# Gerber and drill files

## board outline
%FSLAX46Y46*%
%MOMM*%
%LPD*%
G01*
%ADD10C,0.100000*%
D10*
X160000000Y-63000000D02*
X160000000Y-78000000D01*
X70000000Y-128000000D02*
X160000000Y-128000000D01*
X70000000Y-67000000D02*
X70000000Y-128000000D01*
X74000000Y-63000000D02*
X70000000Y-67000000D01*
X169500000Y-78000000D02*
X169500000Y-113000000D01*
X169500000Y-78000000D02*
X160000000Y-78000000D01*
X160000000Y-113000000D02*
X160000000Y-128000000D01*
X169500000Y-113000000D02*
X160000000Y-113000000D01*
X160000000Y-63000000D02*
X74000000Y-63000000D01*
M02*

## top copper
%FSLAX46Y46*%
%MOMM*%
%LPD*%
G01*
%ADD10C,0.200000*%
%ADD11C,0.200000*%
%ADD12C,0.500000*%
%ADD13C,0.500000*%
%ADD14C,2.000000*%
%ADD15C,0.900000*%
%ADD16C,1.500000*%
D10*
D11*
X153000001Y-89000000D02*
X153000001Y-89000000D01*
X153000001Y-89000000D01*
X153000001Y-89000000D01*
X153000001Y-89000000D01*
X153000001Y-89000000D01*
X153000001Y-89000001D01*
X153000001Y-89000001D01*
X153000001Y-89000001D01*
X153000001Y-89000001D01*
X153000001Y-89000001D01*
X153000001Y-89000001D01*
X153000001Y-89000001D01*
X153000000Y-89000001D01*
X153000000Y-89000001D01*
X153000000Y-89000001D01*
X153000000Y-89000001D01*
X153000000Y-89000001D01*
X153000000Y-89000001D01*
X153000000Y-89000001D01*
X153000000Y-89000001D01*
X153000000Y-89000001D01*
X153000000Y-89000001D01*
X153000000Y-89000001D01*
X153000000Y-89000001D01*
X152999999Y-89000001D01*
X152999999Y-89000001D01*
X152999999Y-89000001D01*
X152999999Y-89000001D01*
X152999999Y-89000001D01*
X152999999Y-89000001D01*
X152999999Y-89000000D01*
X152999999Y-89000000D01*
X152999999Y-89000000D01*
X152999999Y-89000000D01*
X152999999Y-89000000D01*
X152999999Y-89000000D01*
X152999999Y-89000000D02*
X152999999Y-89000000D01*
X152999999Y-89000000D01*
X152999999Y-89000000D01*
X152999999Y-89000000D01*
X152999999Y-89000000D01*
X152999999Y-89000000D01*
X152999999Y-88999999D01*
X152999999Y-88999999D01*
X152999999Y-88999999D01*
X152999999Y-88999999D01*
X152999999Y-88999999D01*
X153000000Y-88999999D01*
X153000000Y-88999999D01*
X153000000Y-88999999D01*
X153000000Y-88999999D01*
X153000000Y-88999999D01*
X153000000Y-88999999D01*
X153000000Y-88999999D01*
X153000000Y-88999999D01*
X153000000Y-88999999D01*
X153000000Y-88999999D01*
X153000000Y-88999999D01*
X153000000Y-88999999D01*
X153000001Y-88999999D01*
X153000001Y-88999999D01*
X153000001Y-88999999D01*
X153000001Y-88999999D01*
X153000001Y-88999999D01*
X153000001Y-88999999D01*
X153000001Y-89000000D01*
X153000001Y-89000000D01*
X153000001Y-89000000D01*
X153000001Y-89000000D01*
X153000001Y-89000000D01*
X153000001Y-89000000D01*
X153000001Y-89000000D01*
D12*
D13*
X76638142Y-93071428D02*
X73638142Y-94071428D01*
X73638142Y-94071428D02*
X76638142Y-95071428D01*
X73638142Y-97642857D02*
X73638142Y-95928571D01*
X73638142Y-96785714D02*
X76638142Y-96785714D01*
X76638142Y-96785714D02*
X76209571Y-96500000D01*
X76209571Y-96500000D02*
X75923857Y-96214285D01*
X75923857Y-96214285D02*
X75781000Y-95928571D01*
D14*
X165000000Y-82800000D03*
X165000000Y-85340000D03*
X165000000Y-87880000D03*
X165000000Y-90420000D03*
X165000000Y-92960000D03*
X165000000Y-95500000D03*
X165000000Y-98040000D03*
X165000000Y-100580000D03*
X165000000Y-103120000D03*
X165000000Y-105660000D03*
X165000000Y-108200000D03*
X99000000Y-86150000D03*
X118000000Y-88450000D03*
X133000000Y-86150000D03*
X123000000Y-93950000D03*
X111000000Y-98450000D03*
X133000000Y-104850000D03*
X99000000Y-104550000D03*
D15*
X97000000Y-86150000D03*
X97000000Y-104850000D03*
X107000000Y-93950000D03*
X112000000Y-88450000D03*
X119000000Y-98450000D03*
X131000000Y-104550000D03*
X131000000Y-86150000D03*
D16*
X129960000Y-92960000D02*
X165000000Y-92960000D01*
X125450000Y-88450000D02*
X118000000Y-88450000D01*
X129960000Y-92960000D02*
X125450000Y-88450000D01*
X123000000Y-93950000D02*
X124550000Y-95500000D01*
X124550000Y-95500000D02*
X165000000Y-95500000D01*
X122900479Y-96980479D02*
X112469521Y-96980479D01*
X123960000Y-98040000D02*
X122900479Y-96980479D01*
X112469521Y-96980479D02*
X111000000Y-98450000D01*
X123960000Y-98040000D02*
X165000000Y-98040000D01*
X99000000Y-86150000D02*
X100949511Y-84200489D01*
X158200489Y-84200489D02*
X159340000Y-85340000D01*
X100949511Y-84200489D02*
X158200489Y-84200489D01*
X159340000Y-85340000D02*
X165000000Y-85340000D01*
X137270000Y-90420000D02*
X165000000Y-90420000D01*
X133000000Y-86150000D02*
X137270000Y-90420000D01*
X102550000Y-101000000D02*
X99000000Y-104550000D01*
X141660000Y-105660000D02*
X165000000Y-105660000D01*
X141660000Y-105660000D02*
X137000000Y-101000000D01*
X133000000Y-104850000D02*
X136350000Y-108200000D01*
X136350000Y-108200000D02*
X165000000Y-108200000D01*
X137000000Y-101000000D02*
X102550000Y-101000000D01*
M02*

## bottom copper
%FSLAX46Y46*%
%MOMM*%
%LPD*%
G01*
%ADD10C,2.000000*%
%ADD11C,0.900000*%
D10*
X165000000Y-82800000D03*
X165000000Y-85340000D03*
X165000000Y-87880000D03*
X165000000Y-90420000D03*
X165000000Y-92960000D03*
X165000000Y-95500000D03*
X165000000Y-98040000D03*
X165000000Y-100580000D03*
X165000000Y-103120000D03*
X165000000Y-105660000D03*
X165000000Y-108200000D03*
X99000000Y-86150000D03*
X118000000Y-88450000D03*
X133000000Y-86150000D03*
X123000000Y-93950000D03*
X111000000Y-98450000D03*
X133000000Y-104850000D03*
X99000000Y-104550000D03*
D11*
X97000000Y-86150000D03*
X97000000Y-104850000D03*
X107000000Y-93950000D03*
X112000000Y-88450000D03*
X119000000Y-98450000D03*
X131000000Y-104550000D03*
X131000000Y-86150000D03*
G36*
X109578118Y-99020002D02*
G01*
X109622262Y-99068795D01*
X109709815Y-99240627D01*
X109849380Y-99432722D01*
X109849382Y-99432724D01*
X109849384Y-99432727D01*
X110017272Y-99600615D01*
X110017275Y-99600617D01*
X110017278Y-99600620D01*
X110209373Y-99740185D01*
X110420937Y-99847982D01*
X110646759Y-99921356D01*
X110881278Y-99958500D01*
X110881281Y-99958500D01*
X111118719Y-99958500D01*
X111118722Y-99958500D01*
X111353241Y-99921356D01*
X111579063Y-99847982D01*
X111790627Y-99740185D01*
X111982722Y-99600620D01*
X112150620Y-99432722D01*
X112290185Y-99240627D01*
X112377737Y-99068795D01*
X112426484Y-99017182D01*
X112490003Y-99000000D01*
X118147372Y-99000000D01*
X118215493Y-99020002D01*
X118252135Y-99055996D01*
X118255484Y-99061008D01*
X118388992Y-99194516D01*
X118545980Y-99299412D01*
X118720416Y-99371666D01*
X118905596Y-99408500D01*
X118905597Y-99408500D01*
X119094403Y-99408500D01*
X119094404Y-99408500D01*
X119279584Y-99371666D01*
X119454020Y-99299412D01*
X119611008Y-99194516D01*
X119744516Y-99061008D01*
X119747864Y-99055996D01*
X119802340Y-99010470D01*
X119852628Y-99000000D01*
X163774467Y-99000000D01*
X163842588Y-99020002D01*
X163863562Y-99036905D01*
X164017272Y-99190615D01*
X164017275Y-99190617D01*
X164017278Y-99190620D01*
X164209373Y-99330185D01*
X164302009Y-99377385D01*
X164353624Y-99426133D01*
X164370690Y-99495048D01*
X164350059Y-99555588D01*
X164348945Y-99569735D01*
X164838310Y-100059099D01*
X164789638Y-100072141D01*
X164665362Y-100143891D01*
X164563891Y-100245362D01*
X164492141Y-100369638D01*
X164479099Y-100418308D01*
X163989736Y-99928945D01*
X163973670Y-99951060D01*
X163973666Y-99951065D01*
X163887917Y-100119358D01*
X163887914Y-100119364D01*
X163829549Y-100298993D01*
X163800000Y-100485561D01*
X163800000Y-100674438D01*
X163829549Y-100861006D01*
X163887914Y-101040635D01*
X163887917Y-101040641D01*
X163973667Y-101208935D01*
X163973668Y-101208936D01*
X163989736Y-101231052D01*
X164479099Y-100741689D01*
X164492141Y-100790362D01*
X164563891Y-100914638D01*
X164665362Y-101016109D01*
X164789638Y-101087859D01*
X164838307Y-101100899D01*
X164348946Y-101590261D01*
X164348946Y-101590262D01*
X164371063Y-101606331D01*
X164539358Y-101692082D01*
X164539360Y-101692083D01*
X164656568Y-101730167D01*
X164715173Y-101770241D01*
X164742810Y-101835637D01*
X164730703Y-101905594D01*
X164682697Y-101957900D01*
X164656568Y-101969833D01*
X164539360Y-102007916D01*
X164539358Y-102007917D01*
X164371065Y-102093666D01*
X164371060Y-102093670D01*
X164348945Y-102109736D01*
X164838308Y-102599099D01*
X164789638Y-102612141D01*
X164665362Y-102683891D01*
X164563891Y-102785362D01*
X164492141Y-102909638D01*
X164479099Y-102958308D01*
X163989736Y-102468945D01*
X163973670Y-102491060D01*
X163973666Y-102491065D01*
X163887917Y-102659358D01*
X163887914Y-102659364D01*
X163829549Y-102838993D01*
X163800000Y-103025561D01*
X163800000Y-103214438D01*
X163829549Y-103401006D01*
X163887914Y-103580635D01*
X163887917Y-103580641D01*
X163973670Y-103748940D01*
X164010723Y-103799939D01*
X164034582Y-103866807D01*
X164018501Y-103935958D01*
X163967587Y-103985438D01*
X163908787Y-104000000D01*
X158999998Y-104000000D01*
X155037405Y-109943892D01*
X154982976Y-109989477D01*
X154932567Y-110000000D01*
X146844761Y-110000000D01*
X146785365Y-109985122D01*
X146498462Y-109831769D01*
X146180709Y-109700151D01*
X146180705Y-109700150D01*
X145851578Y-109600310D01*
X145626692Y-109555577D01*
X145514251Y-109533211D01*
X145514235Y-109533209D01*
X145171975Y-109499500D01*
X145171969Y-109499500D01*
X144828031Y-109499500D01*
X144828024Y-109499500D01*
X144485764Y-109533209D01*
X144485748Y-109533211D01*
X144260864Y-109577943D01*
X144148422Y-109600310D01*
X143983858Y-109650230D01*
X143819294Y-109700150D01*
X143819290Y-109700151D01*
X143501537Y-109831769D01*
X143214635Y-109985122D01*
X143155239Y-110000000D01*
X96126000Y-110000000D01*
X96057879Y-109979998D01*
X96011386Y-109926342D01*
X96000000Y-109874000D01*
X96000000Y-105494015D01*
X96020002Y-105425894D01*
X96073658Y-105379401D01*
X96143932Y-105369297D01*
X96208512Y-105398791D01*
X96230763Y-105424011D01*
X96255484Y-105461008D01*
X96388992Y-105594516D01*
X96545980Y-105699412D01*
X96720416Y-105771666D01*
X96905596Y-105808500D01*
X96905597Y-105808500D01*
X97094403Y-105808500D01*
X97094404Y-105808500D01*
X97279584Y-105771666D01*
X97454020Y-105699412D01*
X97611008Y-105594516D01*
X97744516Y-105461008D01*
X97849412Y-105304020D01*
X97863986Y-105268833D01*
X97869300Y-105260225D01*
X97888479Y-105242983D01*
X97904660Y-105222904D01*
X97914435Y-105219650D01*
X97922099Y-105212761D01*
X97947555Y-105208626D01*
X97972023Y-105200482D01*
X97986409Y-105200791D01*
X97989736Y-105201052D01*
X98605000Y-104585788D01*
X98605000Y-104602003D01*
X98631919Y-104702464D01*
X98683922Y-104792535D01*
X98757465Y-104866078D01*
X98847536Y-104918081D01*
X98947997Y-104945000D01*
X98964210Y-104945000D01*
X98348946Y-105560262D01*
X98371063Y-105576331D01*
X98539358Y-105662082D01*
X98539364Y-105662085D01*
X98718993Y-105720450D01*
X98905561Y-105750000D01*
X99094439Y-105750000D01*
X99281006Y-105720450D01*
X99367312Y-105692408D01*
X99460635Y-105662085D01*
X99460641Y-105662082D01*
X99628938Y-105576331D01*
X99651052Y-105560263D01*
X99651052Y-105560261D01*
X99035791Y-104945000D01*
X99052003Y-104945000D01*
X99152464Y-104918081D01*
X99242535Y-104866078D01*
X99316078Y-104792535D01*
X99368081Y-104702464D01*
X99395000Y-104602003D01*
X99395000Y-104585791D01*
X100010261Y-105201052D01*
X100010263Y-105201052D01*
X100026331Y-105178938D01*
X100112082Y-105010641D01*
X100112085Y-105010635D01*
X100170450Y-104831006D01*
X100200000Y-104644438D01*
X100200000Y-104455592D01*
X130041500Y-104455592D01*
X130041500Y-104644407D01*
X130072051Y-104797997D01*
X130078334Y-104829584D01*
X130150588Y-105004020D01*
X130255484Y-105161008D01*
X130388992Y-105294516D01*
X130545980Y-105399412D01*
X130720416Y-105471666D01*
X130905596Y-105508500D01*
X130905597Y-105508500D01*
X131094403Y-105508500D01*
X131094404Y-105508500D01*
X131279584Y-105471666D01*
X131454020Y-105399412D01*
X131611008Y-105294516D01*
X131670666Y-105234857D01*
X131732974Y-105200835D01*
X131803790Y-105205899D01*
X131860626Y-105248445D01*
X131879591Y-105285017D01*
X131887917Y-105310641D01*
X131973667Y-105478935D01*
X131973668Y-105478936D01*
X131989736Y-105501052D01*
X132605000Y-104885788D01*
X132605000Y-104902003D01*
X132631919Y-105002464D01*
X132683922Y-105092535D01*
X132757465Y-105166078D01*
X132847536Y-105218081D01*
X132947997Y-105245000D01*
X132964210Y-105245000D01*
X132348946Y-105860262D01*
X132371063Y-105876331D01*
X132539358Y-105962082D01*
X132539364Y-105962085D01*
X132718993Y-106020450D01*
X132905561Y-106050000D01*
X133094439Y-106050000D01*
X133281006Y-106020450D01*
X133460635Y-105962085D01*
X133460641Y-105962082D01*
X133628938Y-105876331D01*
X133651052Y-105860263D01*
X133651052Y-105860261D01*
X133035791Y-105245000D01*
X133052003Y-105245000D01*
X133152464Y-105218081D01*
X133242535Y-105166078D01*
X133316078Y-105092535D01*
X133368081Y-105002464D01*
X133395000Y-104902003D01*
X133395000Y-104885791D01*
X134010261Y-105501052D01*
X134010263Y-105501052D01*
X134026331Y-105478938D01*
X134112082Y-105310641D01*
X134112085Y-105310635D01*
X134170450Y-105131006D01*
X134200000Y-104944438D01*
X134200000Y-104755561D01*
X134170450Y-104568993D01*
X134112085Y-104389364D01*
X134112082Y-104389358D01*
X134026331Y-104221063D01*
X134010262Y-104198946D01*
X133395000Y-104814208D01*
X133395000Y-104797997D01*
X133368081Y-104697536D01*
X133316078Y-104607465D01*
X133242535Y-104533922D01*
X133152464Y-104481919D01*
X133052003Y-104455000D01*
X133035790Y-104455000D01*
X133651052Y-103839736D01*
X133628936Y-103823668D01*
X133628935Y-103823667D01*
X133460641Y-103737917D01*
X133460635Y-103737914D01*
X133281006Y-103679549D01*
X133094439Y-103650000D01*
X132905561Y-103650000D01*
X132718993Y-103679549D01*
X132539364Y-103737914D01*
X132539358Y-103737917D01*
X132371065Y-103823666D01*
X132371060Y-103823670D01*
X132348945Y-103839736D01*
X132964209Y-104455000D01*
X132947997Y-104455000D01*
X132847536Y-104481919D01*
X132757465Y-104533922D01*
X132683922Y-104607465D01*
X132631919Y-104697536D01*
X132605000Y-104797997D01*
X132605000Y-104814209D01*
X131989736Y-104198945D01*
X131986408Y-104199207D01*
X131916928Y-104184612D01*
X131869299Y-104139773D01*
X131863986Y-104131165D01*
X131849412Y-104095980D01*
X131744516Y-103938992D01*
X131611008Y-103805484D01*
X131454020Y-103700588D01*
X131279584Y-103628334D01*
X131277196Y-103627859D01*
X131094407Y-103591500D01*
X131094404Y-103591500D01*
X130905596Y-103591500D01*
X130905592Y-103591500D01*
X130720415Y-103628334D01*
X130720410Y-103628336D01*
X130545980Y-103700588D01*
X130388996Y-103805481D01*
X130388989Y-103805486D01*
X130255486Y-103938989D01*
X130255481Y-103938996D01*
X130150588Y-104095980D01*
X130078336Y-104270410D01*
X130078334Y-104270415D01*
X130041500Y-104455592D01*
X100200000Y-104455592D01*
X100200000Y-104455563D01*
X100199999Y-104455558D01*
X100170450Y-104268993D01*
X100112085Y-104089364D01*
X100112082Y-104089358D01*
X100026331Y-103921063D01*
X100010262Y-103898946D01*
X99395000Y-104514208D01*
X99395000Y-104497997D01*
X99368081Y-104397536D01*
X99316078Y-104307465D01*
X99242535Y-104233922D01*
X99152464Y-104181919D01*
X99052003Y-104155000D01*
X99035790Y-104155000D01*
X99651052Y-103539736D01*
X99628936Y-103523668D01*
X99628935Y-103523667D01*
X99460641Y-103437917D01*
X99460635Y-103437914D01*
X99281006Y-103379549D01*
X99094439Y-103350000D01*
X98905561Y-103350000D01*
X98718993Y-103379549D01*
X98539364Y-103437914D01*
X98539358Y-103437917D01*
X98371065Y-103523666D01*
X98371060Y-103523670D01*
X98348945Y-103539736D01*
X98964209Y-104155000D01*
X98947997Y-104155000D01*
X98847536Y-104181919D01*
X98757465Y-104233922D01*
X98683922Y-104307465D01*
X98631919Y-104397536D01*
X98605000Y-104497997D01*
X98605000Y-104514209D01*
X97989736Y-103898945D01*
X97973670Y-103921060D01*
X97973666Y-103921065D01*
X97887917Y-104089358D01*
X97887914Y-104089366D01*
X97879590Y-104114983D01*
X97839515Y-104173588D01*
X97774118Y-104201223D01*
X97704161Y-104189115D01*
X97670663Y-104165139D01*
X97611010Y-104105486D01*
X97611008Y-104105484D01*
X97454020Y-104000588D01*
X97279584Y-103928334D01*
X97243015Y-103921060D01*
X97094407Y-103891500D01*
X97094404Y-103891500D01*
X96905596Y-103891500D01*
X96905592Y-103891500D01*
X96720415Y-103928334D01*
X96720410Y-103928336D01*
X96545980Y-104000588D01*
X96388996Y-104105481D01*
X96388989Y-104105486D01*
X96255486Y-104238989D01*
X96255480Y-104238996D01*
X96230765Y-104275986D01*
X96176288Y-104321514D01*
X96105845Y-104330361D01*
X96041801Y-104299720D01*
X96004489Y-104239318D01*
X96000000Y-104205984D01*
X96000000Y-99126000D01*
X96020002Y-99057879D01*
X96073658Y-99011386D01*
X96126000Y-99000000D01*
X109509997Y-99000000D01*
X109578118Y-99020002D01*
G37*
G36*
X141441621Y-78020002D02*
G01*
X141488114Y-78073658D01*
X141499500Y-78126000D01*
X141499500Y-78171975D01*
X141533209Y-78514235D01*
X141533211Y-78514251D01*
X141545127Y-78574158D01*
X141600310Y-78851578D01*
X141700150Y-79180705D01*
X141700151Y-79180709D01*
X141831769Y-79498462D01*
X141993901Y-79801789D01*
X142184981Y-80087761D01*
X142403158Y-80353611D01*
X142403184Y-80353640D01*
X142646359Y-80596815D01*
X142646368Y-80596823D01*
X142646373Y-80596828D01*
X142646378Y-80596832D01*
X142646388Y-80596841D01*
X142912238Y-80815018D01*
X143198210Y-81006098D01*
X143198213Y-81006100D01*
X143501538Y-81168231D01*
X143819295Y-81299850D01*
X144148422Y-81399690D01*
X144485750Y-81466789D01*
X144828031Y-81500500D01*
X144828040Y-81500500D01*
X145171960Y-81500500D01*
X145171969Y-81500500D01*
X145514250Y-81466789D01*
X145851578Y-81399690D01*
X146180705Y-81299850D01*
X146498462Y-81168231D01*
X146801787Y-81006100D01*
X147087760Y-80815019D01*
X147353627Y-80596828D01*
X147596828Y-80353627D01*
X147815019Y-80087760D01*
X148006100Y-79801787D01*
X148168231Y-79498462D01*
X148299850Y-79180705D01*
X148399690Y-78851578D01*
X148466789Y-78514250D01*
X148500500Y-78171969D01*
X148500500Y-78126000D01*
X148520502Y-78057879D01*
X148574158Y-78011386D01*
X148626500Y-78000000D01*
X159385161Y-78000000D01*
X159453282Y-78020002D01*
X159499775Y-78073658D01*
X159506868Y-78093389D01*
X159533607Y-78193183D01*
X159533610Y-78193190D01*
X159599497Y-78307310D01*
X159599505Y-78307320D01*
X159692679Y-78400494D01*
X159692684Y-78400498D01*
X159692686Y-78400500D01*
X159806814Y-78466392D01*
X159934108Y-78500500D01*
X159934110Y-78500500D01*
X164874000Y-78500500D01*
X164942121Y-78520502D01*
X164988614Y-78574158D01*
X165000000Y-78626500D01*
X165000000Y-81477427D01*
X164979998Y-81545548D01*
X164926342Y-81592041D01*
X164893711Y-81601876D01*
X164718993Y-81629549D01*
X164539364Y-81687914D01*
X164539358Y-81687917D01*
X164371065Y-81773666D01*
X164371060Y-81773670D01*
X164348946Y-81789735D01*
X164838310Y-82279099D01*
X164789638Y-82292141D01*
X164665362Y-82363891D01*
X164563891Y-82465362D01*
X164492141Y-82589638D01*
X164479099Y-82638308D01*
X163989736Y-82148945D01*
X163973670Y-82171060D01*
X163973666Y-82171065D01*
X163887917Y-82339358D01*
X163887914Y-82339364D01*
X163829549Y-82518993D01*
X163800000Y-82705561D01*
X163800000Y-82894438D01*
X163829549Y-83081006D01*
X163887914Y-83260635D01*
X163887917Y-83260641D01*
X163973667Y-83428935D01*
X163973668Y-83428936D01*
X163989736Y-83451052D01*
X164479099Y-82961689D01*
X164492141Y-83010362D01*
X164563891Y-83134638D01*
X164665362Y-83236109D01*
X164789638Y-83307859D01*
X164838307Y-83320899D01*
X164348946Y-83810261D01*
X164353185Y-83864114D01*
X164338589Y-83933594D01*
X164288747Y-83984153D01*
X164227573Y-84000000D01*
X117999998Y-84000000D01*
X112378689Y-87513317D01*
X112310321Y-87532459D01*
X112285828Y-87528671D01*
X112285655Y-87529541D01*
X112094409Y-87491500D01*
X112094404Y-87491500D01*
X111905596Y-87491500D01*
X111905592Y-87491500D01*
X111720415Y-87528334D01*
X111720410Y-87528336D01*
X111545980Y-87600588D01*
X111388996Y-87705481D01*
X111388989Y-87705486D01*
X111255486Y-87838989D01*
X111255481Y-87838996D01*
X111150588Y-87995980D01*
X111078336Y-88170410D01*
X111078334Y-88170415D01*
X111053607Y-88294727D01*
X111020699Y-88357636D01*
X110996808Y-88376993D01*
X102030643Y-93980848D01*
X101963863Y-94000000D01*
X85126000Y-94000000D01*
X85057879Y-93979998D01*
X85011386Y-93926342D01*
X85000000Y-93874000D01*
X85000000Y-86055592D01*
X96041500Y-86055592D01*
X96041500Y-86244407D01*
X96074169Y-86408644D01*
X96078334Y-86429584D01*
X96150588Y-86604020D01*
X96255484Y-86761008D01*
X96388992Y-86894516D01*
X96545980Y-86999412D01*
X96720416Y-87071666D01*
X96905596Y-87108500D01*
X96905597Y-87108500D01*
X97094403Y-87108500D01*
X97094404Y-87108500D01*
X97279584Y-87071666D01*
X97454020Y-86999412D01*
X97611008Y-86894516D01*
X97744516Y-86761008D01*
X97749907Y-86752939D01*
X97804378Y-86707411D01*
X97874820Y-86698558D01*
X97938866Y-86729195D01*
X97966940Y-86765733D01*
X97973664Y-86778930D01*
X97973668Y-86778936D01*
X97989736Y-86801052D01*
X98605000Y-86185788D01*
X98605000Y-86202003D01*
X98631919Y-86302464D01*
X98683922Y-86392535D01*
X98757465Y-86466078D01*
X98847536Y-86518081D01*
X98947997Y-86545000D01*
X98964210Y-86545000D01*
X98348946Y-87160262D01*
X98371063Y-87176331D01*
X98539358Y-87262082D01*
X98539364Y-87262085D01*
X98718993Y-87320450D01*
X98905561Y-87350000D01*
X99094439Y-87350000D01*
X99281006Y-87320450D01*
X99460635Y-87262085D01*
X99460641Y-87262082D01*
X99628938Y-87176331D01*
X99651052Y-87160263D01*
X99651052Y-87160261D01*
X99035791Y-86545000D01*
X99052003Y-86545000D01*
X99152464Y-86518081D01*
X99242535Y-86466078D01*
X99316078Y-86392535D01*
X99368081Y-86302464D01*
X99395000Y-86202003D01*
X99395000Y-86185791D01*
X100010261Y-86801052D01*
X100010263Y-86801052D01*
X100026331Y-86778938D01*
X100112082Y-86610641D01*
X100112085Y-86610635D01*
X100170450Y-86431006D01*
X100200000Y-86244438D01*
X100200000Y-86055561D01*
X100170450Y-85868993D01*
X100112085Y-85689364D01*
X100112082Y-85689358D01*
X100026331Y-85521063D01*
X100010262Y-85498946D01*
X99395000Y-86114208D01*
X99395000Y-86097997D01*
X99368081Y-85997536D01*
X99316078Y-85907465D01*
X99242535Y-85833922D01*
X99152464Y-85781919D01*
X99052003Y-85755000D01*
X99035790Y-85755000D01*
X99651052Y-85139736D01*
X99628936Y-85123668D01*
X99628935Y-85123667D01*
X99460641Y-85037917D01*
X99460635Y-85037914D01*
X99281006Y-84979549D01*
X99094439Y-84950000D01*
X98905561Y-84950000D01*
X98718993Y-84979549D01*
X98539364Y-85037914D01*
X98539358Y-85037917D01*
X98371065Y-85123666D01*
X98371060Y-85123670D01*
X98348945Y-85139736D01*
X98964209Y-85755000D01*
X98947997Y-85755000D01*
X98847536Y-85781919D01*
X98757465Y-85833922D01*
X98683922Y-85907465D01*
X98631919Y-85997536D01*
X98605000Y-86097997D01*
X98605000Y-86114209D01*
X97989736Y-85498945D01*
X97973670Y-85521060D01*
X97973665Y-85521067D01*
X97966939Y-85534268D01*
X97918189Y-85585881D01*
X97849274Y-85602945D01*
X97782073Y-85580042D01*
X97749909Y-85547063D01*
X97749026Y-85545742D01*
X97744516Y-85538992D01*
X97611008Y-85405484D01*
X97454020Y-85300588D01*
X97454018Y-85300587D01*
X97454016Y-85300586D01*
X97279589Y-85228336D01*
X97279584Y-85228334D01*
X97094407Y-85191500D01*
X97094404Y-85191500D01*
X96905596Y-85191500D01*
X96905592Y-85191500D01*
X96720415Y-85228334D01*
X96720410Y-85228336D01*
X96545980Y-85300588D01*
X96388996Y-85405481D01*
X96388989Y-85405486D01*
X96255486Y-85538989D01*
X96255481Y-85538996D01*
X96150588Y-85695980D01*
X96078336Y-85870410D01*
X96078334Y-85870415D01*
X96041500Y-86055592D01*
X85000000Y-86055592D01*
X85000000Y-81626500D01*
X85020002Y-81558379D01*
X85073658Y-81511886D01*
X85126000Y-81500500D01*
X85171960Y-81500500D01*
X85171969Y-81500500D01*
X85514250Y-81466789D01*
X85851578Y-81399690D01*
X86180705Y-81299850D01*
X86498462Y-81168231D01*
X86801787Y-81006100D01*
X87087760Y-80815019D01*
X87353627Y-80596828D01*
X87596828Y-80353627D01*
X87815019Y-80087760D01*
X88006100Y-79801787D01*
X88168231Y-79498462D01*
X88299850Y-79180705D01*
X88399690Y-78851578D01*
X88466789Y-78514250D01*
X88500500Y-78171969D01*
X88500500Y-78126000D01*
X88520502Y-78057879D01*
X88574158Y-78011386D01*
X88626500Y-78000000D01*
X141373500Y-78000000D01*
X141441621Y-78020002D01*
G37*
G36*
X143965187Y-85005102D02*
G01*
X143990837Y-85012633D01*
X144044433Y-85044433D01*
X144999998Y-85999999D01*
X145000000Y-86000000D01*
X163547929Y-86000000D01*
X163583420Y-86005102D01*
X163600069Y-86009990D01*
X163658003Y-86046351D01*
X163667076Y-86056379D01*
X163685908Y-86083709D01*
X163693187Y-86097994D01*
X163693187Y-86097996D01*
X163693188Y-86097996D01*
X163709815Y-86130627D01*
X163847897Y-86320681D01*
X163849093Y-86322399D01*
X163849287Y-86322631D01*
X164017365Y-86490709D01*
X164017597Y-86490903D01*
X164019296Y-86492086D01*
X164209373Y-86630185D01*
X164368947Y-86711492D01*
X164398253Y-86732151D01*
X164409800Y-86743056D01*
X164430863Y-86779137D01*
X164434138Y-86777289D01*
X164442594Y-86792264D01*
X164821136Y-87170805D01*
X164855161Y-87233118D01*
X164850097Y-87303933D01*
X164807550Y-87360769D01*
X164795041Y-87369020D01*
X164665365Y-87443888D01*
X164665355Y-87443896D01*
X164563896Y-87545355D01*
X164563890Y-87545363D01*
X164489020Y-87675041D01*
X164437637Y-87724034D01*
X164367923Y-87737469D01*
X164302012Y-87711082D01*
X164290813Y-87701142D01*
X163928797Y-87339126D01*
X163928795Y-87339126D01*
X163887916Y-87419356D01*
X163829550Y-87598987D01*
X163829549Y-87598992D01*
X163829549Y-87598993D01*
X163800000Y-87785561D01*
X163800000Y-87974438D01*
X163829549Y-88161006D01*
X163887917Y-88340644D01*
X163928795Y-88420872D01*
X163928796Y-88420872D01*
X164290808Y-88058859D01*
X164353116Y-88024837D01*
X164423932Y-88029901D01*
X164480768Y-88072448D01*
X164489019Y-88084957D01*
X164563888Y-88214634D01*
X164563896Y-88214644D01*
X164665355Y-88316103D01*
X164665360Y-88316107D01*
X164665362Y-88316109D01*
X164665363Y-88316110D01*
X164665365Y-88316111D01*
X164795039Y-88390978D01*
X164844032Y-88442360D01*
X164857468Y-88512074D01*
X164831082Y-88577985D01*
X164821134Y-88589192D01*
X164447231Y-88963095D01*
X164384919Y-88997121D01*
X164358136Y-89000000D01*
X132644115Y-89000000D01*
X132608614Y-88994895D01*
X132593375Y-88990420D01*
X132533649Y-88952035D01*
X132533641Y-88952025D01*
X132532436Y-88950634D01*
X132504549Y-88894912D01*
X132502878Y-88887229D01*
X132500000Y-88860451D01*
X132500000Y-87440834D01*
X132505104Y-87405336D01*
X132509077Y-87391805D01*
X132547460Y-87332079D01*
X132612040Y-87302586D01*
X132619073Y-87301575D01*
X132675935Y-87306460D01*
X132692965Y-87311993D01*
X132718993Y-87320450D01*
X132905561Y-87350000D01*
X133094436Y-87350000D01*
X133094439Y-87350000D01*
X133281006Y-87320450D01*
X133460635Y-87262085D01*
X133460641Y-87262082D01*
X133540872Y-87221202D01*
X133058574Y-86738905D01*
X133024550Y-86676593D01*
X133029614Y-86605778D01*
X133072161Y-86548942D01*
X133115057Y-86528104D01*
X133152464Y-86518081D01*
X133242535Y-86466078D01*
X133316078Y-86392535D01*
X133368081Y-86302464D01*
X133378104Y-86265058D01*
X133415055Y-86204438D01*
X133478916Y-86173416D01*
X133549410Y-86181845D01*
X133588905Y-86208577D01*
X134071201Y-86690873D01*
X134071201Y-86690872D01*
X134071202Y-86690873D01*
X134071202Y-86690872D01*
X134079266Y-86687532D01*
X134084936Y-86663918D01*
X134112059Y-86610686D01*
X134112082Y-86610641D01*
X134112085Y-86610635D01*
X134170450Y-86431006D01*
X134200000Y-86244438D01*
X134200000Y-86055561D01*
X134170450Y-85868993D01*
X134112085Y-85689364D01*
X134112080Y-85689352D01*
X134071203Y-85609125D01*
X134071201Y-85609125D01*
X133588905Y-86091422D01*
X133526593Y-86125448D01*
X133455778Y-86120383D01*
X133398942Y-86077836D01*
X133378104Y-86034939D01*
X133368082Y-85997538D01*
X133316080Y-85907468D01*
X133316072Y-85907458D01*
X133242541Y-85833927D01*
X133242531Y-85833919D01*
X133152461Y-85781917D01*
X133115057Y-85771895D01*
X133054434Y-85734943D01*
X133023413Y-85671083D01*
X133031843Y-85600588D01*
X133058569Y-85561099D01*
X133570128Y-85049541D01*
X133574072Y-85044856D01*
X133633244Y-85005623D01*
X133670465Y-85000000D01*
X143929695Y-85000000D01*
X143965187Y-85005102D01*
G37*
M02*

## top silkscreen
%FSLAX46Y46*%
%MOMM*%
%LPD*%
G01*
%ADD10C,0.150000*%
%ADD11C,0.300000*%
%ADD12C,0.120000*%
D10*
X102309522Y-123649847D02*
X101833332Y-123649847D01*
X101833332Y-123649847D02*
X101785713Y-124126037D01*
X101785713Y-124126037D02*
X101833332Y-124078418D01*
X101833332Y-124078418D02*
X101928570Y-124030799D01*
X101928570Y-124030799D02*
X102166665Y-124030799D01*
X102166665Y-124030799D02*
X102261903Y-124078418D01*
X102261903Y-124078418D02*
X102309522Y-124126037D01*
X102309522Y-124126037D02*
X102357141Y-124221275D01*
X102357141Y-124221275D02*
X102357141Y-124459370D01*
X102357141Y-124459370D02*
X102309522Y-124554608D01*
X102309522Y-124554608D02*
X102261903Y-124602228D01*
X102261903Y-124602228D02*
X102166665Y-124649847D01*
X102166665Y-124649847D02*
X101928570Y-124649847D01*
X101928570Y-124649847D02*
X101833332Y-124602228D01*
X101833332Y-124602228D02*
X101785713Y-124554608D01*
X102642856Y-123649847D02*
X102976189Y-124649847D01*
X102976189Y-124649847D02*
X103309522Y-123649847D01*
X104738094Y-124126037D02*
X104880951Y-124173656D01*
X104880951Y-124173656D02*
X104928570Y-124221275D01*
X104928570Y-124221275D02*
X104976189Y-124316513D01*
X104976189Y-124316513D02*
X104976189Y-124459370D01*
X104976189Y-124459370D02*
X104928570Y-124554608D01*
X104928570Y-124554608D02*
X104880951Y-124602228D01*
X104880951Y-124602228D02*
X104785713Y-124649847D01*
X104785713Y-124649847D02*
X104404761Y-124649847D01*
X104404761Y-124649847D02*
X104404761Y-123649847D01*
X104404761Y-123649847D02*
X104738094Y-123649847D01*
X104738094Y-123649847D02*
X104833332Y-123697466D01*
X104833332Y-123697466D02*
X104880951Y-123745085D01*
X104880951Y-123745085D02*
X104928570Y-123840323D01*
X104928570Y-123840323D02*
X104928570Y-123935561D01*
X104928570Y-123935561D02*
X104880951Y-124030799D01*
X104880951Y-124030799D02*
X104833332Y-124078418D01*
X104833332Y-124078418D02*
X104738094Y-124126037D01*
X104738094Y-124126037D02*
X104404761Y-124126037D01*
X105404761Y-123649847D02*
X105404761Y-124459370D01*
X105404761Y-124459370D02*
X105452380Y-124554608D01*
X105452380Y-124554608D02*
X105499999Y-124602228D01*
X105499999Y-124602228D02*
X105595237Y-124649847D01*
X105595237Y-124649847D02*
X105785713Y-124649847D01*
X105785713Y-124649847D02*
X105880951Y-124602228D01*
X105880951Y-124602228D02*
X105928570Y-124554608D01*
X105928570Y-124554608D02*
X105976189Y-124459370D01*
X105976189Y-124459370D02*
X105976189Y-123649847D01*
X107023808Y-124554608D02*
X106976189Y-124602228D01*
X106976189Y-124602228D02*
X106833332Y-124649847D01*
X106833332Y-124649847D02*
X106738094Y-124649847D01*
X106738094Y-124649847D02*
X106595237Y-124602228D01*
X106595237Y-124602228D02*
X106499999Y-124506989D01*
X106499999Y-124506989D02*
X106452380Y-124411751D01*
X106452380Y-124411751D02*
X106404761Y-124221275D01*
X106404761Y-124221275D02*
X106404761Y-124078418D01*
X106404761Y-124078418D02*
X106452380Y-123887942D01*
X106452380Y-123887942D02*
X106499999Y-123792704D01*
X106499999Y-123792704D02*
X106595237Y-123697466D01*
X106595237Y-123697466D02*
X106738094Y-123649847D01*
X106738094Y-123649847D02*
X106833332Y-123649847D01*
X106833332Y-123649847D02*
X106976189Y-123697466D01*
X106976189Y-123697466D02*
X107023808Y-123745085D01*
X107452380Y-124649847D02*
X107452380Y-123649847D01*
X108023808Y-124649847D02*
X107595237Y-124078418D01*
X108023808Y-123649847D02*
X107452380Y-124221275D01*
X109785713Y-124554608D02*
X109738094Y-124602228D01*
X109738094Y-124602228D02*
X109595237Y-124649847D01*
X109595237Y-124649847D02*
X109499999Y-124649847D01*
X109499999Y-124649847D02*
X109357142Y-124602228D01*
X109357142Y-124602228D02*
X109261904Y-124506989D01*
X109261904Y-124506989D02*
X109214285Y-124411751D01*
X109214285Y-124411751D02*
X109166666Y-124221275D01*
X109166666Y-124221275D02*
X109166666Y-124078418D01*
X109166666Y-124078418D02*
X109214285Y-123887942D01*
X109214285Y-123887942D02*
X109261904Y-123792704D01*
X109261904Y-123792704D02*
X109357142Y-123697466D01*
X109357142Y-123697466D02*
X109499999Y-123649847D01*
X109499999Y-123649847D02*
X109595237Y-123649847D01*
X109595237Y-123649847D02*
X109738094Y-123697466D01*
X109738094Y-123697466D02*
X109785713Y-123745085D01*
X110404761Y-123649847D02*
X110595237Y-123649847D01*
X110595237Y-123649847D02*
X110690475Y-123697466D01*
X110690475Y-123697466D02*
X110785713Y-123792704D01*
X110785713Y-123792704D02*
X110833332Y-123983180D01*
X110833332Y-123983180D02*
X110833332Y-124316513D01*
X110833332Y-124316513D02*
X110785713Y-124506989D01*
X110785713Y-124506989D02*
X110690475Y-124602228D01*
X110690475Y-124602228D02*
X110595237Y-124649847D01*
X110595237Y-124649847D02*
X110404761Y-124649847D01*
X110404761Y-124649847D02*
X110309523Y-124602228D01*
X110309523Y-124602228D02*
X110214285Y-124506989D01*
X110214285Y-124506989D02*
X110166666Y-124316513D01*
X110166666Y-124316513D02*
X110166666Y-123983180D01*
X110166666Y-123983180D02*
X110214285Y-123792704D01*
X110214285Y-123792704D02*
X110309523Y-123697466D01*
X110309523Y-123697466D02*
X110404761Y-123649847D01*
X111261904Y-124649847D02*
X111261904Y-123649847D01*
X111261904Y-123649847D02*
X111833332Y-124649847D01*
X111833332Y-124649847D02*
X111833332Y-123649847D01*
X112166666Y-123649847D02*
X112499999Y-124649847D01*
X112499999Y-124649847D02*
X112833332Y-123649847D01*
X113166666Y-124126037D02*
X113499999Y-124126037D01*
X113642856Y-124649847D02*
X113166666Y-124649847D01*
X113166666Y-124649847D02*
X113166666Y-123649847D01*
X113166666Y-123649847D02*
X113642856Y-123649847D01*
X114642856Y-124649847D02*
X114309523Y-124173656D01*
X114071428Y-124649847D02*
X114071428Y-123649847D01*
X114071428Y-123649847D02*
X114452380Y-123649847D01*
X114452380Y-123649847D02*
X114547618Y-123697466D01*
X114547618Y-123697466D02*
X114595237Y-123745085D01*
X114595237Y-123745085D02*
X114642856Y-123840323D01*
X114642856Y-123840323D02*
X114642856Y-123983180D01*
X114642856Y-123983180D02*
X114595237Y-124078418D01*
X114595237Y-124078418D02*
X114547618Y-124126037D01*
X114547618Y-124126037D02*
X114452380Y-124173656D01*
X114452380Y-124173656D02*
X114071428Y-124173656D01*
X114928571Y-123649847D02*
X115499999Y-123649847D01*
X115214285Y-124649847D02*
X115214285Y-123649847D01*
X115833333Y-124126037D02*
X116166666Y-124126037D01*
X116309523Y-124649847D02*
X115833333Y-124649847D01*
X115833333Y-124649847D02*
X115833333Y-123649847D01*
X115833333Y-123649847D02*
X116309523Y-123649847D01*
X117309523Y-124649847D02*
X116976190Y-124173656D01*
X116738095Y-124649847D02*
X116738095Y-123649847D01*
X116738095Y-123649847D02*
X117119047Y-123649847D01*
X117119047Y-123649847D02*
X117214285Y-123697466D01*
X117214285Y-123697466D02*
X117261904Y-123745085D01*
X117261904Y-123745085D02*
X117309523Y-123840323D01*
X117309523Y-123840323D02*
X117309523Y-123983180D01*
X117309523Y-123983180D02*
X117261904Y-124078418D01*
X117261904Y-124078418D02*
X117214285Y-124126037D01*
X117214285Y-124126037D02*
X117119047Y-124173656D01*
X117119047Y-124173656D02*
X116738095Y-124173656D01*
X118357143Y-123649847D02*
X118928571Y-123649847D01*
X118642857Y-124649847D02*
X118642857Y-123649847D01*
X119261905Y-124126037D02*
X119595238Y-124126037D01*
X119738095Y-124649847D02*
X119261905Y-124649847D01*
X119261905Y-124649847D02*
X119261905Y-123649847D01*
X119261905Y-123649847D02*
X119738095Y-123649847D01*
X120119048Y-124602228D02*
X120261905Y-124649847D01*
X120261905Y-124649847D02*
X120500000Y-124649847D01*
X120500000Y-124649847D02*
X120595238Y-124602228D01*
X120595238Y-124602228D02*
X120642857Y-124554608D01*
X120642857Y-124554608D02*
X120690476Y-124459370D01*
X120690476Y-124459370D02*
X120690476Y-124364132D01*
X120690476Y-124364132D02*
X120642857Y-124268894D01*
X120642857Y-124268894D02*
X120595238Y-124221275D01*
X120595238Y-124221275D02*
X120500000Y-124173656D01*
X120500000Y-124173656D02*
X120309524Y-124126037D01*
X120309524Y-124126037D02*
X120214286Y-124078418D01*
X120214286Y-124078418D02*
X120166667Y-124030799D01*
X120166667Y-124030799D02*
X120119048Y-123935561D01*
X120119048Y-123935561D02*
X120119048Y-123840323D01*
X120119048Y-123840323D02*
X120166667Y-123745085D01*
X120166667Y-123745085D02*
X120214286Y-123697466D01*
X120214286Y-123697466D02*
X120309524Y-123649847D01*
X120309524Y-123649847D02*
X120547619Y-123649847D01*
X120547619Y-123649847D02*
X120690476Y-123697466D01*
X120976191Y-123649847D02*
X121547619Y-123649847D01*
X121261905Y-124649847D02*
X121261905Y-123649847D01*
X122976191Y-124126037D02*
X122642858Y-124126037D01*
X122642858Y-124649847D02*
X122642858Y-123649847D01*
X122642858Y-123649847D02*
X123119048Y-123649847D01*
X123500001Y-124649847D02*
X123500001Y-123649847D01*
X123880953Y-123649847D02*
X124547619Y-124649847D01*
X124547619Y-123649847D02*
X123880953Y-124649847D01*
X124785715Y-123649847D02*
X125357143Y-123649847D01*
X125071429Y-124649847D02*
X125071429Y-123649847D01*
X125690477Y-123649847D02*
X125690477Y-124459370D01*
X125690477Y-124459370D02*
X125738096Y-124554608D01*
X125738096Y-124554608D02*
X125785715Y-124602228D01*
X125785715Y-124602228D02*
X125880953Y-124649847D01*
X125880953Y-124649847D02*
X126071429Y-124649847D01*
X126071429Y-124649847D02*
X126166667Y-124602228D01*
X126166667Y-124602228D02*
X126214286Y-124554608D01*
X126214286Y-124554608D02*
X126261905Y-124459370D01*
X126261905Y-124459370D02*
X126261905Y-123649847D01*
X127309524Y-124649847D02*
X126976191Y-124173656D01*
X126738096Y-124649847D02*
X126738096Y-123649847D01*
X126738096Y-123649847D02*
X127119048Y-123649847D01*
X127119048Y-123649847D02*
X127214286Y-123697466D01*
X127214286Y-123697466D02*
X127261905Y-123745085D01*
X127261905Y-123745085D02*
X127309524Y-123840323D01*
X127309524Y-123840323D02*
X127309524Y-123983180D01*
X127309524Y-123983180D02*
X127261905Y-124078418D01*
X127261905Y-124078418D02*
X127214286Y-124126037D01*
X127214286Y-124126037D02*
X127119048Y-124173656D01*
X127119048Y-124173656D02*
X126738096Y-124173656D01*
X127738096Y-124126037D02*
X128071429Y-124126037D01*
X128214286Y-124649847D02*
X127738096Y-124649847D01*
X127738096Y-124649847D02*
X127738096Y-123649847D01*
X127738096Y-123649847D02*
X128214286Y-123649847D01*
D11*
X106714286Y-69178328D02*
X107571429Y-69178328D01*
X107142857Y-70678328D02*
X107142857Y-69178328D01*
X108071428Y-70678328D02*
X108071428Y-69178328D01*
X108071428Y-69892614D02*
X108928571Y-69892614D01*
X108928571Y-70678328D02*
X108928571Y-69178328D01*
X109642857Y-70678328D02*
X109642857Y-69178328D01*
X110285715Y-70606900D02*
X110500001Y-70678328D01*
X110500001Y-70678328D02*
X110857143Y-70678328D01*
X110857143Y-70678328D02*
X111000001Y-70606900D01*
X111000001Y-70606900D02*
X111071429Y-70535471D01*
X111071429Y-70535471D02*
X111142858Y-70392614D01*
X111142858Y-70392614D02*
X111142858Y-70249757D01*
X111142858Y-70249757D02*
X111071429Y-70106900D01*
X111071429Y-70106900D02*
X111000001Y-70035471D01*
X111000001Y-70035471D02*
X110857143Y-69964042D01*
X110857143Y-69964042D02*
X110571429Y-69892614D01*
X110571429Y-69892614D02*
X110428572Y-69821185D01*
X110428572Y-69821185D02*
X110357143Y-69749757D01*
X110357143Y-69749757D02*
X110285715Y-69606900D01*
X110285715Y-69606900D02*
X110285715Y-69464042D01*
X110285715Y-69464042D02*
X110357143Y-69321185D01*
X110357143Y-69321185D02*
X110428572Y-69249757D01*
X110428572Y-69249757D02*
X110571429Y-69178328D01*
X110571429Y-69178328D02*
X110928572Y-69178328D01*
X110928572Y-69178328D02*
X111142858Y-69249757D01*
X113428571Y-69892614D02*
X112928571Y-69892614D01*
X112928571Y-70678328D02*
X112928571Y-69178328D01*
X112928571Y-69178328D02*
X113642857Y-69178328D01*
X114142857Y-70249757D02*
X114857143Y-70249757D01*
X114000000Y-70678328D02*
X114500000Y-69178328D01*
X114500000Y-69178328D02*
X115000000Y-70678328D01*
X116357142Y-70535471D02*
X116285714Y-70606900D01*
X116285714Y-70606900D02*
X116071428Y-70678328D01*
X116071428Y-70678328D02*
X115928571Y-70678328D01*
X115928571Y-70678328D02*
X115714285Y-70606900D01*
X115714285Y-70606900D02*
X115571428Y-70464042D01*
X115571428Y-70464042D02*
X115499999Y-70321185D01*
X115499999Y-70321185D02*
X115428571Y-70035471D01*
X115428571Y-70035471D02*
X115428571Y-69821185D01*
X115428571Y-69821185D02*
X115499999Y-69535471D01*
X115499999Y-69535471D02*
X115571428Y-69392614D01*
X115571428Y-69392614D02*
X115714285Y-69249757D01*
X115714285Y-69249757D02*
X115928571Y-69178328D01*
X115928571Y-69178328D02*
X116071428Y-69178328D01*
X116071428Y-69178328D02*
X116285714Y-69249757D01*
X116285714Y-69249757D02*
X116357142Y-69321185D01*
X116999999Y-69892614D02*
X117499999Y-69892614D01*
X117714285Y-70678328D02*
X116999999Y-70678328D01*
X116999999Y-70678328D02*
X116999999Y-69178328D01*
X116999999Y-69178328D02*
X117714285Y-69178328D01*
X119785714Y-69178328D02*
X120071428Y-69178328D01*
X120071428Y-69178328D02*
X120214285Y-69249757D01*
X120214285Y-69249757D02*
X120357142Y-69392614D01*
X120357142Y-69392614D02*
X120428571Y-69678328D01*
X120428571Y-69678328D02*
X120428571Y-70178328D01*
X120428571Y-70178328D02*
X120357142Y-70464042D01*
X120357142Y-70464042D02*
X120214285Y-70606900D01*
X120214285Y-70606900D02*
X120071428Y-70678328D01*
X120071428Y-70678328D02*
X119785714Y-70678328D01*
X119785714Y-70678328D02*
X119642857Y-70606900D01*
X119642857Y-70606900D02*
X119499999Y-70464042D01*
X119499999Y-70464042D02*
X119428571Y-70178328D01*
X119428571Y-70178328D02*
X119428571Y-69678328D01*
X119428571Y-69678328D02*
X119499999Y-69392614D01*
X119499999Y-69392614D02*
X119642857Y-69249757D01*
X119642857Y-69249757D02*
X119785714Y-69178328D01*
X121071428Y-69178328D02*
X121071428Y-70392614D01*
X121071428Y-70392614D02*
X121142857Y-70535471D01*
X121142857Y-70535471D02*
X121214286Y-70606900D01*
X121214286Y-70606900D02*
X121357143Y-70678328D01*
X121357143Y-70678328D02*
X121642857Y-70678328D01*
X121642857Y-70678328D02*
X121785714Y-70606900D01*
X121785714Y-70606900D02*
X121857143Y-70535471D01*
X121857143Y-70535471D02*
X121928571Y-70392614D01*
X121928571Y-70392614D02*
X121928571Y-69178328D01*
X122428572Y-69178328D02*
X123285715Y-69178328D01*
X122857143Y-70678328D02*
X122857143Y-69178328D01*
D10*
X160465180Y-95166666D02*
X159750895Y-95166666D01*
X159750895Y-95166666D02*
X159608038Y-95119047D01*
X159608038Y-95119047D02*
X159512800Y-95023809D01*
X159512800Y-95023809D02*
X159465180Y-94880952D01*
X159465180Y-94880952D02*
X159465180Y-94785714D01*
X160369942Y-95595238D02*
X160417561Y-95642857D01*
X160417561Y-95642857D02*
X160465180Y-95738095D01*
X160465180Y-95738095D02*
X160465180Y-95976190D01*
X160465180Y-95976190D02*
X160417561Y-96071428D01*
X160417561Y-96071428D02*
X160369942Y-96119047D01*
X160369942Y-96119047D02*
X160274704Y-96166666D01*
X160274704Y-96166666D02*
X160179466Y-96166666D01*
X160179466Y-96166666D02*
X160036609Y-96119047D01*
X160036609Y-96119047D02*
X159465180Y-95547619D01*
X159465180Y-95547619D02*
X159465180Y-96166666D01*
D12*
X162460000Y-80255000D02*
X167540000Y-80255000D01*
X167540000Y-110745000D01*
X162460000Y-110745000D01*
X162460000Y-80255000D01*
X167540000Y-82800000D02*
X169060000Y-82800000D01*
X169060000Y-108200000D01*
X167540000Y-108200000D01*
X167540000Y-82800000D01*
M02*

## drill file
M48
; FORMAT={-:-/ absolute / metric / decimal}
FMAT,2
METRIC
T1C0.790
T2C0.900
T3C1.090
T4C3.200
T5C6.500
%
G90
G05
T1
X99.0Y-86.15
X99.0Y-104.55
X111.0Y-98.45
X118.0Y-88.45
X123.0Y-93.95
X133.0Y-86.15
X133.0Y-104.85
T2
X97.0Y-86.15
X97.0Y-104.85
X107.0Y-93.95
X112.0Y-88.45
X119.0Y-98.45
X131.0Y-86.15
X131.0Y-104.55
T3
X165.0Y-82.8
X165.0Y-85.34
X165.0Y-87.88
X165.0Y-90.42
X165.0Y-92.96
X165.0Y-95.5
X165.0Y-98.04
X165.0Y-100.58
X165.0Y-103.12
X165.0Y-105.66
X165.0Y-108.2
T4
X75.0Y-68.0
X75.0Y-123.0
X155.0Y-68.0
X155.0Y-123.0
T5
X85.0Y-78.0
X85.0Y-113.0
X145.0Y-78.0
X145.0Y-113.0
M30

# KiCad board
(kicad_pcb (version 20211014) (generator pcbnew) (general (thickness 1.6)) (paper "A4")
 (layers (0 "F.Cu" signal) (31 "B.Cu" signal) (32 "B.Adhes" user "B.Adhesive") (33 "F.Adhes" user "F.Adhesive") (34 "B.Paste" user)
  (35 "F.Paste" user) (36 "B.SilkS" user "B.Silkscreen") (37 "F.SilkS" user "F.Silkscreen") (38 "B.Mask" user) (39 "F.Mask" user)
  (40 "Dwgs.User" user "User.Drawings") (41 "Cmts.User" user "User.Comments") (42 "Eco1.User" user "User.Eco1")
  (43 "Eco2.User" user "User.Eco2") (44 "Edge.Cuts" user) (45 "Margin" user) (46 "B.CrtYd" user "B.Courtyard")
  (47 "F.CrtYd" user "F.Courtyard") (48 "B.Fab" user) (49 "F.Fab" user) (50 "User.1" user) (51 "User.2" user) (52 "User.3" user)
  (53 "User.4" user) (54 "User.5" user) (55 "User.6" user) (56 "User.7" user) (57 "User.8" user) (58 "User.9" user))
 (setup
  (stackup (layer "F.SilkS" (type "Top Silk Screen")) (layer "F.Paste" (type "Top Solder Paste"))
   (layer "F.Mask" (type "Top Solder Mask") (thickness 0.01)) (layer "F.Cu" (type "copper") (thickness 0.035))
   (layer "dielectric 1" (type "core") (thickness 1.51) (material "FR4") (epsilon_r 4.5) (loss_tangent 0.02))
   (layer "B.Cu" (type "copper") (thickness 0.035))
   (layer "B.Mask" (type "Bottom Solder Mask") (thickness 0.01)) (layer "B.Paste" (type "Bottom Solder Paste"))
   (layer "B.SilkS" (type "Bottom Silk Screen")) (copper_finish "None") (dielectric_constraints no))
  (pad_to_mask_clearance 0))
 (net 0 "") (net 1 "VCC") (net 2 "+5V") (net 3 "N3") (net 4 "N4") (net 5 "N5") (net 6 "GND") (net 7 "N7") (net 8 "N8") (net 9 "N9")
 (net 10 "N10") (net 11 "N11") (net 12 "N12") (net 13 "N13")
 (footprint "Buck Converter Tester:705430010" (layer "F.Cu") (at 165 95.5 -90)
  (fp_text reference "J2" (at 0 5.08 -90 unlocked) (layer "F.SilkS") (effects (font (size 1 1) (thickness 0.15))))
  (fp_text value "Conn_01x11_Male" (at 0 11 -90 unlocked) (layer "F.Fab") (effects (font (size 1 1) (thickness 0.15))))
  (fp_rect (start -15.245 -2.54) (end 15.245 2.54) (layer "F.SilkS") (width 0.12) (fill none))
  (fp_rect (start -12.7 -2.54) (end 12.7 -4.06) (layer "F.SilkS") (width 0.12) (fill none))
  (pad "1" thru_hole circle (at -12.7 0 270) (size 2 2) (drill 1.09) (layers *.Cu *.Mask) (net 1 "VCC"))
  (pad "2" thru_hole circle (at -10.16 0 270) (size 2 2) (drill 1.09) (layers *.Cu *.Mask) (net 1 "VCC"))
  (pad "3" thru_hole circle (at -7.62 0 270) (size 2 2) (drill 1.09) (layers *.Cu *.Mask) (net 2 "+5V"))
  (pad "4" thru_hole circle (at -5.08 0 270) (size 2 2) (drill 1.09) (layers *.Cu *.Mask) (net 2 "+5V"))
  (pad "5" thru_hole circle (at -2.54 0 270) (size 2 2) (drill 1.09) (layers *.Cu *.Mask) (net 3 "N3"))
  (pad "6" thru_hole circle (at 0 0 270) (size 2 2) (drill 1.09) (layers *.Cu *.Mask) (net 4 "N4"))
  (pad "7" thru_hole circle (at 2.54 0 270) (size 2 2) (drill 1.09) (layers *.Cu *.Mask) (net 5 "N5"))
  (pad "8" thru_hole circle (at 5.08 0 270) (size 2 2) (drill 1.09) (layers *.Cu *.Mask) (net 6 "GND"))
  (pad "9" thru_hole circle (at 7.62 0 270) (size 2 2) (drill 1.09) (layers *.Cu *.Mask) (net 6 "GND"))
  (pad "10" thru_hole circle (at 10.16 0 270) (size 2 2) (drill 1.09) (layers *.Cu *.Mask) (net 6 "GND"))
  (pad "11" thru_hole circle (at 12.7 0 270) (size 2 2) (drill 1.09) (layers *.Cu *.Mask) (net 6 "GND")))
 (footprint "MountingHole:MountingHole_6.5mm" (layer "F.Cu") (at 145 113)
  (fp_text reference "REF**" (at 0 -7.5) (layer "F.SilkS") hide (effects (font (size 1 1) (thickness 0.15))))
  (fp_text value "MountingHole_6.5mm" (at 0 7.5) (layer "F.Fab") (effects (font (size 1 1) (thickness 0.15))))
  (pad "" np_thru_hole circle (at 0 0) (size 6.5 6.5) (drill 6.5) (layers *.Cu *.Mask)))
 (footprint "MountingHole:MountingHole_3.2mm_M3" (layer "F.Cu") (at 75 68)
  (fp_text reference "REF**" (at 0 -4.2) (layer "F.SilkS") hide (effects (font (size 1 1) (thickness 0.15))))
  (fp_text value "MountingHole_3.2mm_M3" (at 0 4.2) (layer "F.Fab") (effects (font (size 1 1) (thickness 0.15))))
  (pad "" np_thru_hole circle (at 0 0) (size 3.2 3.2) (drill 3.2) (layers *.Cu *.Mask)))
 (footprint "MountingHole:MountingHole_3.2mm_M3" (layer "F.Cu") (at 75 123)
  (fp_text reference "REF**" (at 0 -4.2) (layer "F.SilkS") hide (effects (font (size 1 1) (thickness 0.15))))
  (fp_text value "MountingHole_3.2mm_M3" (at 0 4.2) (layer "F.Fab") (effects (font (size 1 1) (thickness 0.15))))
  (pad "" np_thru_hole circle (at 0 0) (size 3.2 3.2) (drill 3.2) (layers *.Cu *.Mask)))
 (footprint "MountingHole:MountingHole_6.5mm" (layer "F.Cu") (at 85 78)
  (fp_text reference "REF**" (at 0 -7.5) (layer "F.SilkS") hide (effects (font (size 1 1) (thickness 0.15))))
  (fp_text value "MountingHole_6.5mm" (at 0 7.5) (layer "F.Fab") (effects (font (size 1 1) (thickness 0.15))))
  (pad "" np_thru_hole circle (at 0 0) (size 6.5 6.5) (drill 6.5) (layers *.Cu *.Mask)))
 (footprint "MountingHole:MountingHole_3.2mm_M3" (layer "F.Cu") (at 155 123)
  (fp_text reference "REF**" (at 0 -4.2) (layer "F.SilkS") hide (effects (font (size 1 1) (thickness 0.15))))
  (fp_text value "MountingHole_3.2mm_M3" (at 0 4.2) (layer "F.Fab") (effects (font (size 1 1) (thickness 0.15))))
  (pad "" np_thru_hole circle (at 0 0) (size 3.2 3.2) (drill 3.2) (layers *.Cu *.Mask)))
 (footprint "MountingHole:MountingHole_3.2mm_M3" (layer "F.Cu") (at 155 68)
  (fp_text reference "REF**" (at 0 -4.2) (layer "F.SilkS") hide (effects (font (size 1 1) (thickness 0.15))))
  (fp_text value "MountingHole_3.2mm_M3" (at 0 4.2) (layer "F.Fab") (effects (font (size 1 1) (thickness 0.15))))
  (pad "" np_thru_hole circle (at 0 0) (size 3.2 3.2) (drill 3.2) (layers *.Cu *.Mask)))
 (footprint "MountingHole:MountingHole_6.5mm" (layer "F.Cu") (at 85 113)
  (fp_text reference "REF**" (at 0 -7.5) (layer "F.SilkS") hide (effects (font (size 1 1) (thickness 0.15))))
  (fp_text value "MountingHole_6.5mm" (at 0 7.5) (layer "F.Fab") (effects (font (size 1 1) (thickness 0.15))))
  (pad "" np_thru_hole circle (at 0 0) (size 6.5 6.5) (drill 6.5) (layers *.Cu *.Mask)))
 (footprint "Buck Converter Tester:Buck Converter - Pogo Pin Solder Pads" (layer "F.Cu") (at 133 86.15 180)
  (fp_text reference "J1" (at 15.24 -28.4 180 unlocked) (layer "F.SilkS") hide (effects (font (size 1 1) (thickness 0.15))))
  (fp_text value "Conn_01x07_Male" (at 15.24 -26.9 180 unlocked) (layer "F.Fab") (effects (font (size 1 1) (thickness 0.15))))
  (pad "1" thru_hole circle (at 34 0 180) (size 2 2) (drill 0.79) (layers *.Cu *.Mask) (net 1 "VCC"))
  (pad "2" thru_hole circle (at 15 -2.3 180) (size 2 2) (drill 0.79) (layers *.Cu *.Mask) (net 3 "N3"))
  (pad "3" thru_hole circle (at 0 0 180) (size 2 2) (drill 0.79) (layers *.Cu *.Mask) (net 2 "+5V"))
  (pad "4" thru_hole circle (at 10 -7.8 180) (size 2 2) (drill 0.79) (layers *.Cu *.Mask) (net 4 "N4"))
  (pad "5" thru_hole circle (at 22 -12.3 180) (size 2 2) (drill 0.79) (layers *.Cu *.Mask) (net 5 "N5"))
  (pad "6" thru_hole circle (at 0 -18.7 180) (size 2 2) (drill 0.79) (layers *.Cu *.Mask) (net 6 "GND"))
  (pad "7" thru_hole circle (at 34 -18.4 180) (size 2 2) (drill 0.79) (layers *.Cu *.Mask) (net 6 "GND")))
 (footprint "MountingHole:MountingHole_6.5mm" (layer "F.Cu") (at 145 78)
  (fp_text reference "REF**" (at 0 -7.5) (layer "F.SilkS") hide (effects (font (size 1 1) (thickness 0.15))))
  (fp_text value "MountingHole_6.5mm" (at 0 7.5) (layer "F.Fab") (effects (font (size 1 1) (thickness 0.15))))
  (pad "" np_thru_hole circle (at 0 0) (size 6.5 6.5) (drill 6.5) (layers *.Cu *.Mask)))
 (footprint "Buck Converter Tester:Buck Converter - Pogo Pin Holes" (layer "B.Cu") (at 97 86.15)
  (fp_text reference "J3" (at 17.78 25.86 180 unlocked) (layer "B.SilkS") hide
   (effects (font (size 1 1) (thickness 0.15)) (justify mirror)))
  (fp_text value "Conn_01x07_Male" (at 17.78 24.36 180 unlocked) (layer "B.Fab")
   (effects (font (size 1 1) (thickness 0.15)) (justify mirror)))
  (pad "1" thru_hole circle (at 0 0) (size 0.9 0.9) (drill 0.9) (layers *.Cu *.Mask) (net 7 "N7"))
  (pad "2" thru_hole circle (at 0 18.7) (size 0.9 0.9) (drill 0.9) (layers *.Cu *.Mask) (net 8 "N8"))
  (pad "3" thru_hole circle (at 10 7.8) (size 0.9 0.9) (drill 0.9) (layers *.Cu *.Mask) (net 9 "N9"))
  (pad "4" thru_hole circle (at 15 2.3) (size 0.9 0.9) (drill 0.9) (layers *.Cu *.Mask) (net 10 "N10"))
  (pad "5" thru_hole circle (at 22 12.3) (size 0.9 0.9) (drill 0.9) (layers *.Cu *.Mask) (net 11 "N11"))
  (pad "6" thru_hole circle (at 34 18.4) (size 0.9 0.9) (drill 0.9) (layers *.Cu *.Mask) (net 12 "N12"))
  (pad "7" thru_hole circle (at 34 0) (size 0.9 0.9) (drill 0.9) (layers *.Cu *.Mask) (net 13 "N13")))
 (gr_circle (center 153 89) (end 153 89) (layer "F.Cu") (width 0.2) (fill none))
 (gr_line (start 160 63) (end 160 78) (layer "Edge.Cuts") (width 0.1))
 (gr_line (start 70 128) (end 160 128) (layer "Edge.Cuts") (width 0.1))
 (gr_line (start 70 67) (end 70 128) (layer "Edge.Cuts") (width 0.1))
 (gr_line (start 74 63) (end 70 67) (layer "Edge.Cuts") (width 0.1))
 (gr_line (start 169.5 78) (end 169.5 113) (layer "Edge.Cuts") (width 0.1))
 (gr_line (start 169.5 78) (end 160 78) (layer "Edge.Cuts") (width 0.1))
 (gr_line (start 160 113) (end 160 128) (layer "Edge.Cuts") (width 0.1))
 (gr_line (start 169.5 113) (end 160 113) (layer "Edge.Cuts") (width 0.1))
 (gr_line (start 160 63) (end 74 63) (layer "Edge.Cuts") (width 0.1))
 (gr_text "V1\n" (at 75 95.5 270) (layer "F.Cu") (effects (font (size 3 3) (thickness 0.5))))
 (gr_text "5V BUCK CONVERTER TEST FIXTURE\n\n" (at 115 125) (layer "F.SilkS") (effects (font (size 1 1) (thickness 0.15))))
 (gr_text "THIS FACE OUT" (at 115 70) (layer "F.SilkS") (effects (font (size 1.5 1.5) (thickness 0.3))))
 (segment (start 129.96 92.96) (end 165 92.96) (width 1.5) (layer "F.Cu") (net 3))
 (segment (start 125.45 88.45) (end 118 88.45) (width 1.5) (layer "F.Cu") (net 3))
 (segment (start 129.96 92.96) (end 125.45 88.45) (width 1.5) (layer "F.Cu") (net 3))
 (segment (start 123 93.95) (end 124.55 95.5) (width 1.5) (layer "F.Cu") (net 4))
 (segment (start 124.55 95.5) (end 165 95.5) (width 1.5) (layer "F.Cu") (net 4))
 (segment (start 122.900479 96.980479) (end 112.469521 96.980479) (width 1.5) (layer "F.Cu") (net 5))
 (segment (start 123.96 98.04) (end 122.900479 96.980479) (width 1.5) (layer "F.Cu") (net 5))
 (segment (start 112.469521 96.980479) (end 111 98.45) (width 1.5) (layer "F.Cu") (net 5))
 (segment (start 123.96 98.04) (end 165 98.04) (width 1.5) (layer "F.Cu") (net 5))
 (segment (start 99 86.15) (end 100.949511 84.200489) (width 1.5) (layer "F.Cu") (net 1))
 (segment (start 158.200489 84.200489) (end 159.34 85.34) (width 1.5) (layer "F.Cu") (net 1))
 (segment (start 100.949511 84.200489) (end 158.200489 84.200489) (width 1.5) (layer "F.Cu") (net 1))
 (segment (start 159.34 85.34) (end 165 85.34) (width 1.5) (layer "F.Cu") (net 1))
 (segment (start 137.27 90.42) (end 165 90.42) (width 1.5) (layer "F.Cu") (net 2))
 (segment (start 133 86.15) (end 137.27 90.42) (width 1.5) (layer "F.Cu") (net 2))
 (segment (start 102.55 101) (end 99 104.55) (width 1.5) (layer "F.Cu") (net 6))
 (segment (start 141.66 105.66) (end 165 105.66) (width 1.5) (layer "F.Cu") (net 6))
 (segment (start 141.66 105.66) (end 137 101) (width 1.5) (layer "F.Cu") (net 6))
 (segment (start 133 104.85) (end 136.35 108.2) (width 1.5) (layer "F.Cu") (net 6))
 (segment (start 136.35 108.2) (end 165 108.2) (width 1.5) (layer "F.Cu") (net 6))
 (segment (start 137 101) (end 102.55 101) (width 1.5) (layer "F.Cu") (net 6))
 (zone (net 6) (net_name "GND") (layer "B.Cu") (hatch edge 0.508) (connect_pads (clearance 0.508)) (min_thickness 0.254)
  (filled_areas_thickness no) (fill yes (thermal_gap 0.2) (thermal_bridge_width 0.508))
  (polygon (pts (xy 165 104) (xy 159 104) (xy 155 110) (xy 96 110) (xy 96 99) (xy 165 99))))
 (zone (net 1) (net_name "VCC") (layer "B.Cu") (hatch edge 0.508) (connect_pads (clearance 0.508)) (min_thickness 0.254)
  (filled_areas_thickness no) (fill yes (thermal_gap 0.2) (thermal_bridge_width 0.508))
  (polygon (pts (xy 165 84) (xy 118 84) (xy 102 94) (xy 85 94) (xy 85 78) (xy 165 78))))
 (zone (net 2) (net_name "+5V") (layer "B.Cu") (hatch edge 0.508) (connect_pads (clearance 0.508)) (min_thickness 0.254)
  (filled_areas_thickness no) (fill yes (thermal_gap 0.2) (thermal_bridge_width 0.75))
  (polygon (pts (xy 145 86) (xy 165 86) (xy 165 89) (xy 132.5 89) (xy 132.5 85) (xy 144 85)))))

